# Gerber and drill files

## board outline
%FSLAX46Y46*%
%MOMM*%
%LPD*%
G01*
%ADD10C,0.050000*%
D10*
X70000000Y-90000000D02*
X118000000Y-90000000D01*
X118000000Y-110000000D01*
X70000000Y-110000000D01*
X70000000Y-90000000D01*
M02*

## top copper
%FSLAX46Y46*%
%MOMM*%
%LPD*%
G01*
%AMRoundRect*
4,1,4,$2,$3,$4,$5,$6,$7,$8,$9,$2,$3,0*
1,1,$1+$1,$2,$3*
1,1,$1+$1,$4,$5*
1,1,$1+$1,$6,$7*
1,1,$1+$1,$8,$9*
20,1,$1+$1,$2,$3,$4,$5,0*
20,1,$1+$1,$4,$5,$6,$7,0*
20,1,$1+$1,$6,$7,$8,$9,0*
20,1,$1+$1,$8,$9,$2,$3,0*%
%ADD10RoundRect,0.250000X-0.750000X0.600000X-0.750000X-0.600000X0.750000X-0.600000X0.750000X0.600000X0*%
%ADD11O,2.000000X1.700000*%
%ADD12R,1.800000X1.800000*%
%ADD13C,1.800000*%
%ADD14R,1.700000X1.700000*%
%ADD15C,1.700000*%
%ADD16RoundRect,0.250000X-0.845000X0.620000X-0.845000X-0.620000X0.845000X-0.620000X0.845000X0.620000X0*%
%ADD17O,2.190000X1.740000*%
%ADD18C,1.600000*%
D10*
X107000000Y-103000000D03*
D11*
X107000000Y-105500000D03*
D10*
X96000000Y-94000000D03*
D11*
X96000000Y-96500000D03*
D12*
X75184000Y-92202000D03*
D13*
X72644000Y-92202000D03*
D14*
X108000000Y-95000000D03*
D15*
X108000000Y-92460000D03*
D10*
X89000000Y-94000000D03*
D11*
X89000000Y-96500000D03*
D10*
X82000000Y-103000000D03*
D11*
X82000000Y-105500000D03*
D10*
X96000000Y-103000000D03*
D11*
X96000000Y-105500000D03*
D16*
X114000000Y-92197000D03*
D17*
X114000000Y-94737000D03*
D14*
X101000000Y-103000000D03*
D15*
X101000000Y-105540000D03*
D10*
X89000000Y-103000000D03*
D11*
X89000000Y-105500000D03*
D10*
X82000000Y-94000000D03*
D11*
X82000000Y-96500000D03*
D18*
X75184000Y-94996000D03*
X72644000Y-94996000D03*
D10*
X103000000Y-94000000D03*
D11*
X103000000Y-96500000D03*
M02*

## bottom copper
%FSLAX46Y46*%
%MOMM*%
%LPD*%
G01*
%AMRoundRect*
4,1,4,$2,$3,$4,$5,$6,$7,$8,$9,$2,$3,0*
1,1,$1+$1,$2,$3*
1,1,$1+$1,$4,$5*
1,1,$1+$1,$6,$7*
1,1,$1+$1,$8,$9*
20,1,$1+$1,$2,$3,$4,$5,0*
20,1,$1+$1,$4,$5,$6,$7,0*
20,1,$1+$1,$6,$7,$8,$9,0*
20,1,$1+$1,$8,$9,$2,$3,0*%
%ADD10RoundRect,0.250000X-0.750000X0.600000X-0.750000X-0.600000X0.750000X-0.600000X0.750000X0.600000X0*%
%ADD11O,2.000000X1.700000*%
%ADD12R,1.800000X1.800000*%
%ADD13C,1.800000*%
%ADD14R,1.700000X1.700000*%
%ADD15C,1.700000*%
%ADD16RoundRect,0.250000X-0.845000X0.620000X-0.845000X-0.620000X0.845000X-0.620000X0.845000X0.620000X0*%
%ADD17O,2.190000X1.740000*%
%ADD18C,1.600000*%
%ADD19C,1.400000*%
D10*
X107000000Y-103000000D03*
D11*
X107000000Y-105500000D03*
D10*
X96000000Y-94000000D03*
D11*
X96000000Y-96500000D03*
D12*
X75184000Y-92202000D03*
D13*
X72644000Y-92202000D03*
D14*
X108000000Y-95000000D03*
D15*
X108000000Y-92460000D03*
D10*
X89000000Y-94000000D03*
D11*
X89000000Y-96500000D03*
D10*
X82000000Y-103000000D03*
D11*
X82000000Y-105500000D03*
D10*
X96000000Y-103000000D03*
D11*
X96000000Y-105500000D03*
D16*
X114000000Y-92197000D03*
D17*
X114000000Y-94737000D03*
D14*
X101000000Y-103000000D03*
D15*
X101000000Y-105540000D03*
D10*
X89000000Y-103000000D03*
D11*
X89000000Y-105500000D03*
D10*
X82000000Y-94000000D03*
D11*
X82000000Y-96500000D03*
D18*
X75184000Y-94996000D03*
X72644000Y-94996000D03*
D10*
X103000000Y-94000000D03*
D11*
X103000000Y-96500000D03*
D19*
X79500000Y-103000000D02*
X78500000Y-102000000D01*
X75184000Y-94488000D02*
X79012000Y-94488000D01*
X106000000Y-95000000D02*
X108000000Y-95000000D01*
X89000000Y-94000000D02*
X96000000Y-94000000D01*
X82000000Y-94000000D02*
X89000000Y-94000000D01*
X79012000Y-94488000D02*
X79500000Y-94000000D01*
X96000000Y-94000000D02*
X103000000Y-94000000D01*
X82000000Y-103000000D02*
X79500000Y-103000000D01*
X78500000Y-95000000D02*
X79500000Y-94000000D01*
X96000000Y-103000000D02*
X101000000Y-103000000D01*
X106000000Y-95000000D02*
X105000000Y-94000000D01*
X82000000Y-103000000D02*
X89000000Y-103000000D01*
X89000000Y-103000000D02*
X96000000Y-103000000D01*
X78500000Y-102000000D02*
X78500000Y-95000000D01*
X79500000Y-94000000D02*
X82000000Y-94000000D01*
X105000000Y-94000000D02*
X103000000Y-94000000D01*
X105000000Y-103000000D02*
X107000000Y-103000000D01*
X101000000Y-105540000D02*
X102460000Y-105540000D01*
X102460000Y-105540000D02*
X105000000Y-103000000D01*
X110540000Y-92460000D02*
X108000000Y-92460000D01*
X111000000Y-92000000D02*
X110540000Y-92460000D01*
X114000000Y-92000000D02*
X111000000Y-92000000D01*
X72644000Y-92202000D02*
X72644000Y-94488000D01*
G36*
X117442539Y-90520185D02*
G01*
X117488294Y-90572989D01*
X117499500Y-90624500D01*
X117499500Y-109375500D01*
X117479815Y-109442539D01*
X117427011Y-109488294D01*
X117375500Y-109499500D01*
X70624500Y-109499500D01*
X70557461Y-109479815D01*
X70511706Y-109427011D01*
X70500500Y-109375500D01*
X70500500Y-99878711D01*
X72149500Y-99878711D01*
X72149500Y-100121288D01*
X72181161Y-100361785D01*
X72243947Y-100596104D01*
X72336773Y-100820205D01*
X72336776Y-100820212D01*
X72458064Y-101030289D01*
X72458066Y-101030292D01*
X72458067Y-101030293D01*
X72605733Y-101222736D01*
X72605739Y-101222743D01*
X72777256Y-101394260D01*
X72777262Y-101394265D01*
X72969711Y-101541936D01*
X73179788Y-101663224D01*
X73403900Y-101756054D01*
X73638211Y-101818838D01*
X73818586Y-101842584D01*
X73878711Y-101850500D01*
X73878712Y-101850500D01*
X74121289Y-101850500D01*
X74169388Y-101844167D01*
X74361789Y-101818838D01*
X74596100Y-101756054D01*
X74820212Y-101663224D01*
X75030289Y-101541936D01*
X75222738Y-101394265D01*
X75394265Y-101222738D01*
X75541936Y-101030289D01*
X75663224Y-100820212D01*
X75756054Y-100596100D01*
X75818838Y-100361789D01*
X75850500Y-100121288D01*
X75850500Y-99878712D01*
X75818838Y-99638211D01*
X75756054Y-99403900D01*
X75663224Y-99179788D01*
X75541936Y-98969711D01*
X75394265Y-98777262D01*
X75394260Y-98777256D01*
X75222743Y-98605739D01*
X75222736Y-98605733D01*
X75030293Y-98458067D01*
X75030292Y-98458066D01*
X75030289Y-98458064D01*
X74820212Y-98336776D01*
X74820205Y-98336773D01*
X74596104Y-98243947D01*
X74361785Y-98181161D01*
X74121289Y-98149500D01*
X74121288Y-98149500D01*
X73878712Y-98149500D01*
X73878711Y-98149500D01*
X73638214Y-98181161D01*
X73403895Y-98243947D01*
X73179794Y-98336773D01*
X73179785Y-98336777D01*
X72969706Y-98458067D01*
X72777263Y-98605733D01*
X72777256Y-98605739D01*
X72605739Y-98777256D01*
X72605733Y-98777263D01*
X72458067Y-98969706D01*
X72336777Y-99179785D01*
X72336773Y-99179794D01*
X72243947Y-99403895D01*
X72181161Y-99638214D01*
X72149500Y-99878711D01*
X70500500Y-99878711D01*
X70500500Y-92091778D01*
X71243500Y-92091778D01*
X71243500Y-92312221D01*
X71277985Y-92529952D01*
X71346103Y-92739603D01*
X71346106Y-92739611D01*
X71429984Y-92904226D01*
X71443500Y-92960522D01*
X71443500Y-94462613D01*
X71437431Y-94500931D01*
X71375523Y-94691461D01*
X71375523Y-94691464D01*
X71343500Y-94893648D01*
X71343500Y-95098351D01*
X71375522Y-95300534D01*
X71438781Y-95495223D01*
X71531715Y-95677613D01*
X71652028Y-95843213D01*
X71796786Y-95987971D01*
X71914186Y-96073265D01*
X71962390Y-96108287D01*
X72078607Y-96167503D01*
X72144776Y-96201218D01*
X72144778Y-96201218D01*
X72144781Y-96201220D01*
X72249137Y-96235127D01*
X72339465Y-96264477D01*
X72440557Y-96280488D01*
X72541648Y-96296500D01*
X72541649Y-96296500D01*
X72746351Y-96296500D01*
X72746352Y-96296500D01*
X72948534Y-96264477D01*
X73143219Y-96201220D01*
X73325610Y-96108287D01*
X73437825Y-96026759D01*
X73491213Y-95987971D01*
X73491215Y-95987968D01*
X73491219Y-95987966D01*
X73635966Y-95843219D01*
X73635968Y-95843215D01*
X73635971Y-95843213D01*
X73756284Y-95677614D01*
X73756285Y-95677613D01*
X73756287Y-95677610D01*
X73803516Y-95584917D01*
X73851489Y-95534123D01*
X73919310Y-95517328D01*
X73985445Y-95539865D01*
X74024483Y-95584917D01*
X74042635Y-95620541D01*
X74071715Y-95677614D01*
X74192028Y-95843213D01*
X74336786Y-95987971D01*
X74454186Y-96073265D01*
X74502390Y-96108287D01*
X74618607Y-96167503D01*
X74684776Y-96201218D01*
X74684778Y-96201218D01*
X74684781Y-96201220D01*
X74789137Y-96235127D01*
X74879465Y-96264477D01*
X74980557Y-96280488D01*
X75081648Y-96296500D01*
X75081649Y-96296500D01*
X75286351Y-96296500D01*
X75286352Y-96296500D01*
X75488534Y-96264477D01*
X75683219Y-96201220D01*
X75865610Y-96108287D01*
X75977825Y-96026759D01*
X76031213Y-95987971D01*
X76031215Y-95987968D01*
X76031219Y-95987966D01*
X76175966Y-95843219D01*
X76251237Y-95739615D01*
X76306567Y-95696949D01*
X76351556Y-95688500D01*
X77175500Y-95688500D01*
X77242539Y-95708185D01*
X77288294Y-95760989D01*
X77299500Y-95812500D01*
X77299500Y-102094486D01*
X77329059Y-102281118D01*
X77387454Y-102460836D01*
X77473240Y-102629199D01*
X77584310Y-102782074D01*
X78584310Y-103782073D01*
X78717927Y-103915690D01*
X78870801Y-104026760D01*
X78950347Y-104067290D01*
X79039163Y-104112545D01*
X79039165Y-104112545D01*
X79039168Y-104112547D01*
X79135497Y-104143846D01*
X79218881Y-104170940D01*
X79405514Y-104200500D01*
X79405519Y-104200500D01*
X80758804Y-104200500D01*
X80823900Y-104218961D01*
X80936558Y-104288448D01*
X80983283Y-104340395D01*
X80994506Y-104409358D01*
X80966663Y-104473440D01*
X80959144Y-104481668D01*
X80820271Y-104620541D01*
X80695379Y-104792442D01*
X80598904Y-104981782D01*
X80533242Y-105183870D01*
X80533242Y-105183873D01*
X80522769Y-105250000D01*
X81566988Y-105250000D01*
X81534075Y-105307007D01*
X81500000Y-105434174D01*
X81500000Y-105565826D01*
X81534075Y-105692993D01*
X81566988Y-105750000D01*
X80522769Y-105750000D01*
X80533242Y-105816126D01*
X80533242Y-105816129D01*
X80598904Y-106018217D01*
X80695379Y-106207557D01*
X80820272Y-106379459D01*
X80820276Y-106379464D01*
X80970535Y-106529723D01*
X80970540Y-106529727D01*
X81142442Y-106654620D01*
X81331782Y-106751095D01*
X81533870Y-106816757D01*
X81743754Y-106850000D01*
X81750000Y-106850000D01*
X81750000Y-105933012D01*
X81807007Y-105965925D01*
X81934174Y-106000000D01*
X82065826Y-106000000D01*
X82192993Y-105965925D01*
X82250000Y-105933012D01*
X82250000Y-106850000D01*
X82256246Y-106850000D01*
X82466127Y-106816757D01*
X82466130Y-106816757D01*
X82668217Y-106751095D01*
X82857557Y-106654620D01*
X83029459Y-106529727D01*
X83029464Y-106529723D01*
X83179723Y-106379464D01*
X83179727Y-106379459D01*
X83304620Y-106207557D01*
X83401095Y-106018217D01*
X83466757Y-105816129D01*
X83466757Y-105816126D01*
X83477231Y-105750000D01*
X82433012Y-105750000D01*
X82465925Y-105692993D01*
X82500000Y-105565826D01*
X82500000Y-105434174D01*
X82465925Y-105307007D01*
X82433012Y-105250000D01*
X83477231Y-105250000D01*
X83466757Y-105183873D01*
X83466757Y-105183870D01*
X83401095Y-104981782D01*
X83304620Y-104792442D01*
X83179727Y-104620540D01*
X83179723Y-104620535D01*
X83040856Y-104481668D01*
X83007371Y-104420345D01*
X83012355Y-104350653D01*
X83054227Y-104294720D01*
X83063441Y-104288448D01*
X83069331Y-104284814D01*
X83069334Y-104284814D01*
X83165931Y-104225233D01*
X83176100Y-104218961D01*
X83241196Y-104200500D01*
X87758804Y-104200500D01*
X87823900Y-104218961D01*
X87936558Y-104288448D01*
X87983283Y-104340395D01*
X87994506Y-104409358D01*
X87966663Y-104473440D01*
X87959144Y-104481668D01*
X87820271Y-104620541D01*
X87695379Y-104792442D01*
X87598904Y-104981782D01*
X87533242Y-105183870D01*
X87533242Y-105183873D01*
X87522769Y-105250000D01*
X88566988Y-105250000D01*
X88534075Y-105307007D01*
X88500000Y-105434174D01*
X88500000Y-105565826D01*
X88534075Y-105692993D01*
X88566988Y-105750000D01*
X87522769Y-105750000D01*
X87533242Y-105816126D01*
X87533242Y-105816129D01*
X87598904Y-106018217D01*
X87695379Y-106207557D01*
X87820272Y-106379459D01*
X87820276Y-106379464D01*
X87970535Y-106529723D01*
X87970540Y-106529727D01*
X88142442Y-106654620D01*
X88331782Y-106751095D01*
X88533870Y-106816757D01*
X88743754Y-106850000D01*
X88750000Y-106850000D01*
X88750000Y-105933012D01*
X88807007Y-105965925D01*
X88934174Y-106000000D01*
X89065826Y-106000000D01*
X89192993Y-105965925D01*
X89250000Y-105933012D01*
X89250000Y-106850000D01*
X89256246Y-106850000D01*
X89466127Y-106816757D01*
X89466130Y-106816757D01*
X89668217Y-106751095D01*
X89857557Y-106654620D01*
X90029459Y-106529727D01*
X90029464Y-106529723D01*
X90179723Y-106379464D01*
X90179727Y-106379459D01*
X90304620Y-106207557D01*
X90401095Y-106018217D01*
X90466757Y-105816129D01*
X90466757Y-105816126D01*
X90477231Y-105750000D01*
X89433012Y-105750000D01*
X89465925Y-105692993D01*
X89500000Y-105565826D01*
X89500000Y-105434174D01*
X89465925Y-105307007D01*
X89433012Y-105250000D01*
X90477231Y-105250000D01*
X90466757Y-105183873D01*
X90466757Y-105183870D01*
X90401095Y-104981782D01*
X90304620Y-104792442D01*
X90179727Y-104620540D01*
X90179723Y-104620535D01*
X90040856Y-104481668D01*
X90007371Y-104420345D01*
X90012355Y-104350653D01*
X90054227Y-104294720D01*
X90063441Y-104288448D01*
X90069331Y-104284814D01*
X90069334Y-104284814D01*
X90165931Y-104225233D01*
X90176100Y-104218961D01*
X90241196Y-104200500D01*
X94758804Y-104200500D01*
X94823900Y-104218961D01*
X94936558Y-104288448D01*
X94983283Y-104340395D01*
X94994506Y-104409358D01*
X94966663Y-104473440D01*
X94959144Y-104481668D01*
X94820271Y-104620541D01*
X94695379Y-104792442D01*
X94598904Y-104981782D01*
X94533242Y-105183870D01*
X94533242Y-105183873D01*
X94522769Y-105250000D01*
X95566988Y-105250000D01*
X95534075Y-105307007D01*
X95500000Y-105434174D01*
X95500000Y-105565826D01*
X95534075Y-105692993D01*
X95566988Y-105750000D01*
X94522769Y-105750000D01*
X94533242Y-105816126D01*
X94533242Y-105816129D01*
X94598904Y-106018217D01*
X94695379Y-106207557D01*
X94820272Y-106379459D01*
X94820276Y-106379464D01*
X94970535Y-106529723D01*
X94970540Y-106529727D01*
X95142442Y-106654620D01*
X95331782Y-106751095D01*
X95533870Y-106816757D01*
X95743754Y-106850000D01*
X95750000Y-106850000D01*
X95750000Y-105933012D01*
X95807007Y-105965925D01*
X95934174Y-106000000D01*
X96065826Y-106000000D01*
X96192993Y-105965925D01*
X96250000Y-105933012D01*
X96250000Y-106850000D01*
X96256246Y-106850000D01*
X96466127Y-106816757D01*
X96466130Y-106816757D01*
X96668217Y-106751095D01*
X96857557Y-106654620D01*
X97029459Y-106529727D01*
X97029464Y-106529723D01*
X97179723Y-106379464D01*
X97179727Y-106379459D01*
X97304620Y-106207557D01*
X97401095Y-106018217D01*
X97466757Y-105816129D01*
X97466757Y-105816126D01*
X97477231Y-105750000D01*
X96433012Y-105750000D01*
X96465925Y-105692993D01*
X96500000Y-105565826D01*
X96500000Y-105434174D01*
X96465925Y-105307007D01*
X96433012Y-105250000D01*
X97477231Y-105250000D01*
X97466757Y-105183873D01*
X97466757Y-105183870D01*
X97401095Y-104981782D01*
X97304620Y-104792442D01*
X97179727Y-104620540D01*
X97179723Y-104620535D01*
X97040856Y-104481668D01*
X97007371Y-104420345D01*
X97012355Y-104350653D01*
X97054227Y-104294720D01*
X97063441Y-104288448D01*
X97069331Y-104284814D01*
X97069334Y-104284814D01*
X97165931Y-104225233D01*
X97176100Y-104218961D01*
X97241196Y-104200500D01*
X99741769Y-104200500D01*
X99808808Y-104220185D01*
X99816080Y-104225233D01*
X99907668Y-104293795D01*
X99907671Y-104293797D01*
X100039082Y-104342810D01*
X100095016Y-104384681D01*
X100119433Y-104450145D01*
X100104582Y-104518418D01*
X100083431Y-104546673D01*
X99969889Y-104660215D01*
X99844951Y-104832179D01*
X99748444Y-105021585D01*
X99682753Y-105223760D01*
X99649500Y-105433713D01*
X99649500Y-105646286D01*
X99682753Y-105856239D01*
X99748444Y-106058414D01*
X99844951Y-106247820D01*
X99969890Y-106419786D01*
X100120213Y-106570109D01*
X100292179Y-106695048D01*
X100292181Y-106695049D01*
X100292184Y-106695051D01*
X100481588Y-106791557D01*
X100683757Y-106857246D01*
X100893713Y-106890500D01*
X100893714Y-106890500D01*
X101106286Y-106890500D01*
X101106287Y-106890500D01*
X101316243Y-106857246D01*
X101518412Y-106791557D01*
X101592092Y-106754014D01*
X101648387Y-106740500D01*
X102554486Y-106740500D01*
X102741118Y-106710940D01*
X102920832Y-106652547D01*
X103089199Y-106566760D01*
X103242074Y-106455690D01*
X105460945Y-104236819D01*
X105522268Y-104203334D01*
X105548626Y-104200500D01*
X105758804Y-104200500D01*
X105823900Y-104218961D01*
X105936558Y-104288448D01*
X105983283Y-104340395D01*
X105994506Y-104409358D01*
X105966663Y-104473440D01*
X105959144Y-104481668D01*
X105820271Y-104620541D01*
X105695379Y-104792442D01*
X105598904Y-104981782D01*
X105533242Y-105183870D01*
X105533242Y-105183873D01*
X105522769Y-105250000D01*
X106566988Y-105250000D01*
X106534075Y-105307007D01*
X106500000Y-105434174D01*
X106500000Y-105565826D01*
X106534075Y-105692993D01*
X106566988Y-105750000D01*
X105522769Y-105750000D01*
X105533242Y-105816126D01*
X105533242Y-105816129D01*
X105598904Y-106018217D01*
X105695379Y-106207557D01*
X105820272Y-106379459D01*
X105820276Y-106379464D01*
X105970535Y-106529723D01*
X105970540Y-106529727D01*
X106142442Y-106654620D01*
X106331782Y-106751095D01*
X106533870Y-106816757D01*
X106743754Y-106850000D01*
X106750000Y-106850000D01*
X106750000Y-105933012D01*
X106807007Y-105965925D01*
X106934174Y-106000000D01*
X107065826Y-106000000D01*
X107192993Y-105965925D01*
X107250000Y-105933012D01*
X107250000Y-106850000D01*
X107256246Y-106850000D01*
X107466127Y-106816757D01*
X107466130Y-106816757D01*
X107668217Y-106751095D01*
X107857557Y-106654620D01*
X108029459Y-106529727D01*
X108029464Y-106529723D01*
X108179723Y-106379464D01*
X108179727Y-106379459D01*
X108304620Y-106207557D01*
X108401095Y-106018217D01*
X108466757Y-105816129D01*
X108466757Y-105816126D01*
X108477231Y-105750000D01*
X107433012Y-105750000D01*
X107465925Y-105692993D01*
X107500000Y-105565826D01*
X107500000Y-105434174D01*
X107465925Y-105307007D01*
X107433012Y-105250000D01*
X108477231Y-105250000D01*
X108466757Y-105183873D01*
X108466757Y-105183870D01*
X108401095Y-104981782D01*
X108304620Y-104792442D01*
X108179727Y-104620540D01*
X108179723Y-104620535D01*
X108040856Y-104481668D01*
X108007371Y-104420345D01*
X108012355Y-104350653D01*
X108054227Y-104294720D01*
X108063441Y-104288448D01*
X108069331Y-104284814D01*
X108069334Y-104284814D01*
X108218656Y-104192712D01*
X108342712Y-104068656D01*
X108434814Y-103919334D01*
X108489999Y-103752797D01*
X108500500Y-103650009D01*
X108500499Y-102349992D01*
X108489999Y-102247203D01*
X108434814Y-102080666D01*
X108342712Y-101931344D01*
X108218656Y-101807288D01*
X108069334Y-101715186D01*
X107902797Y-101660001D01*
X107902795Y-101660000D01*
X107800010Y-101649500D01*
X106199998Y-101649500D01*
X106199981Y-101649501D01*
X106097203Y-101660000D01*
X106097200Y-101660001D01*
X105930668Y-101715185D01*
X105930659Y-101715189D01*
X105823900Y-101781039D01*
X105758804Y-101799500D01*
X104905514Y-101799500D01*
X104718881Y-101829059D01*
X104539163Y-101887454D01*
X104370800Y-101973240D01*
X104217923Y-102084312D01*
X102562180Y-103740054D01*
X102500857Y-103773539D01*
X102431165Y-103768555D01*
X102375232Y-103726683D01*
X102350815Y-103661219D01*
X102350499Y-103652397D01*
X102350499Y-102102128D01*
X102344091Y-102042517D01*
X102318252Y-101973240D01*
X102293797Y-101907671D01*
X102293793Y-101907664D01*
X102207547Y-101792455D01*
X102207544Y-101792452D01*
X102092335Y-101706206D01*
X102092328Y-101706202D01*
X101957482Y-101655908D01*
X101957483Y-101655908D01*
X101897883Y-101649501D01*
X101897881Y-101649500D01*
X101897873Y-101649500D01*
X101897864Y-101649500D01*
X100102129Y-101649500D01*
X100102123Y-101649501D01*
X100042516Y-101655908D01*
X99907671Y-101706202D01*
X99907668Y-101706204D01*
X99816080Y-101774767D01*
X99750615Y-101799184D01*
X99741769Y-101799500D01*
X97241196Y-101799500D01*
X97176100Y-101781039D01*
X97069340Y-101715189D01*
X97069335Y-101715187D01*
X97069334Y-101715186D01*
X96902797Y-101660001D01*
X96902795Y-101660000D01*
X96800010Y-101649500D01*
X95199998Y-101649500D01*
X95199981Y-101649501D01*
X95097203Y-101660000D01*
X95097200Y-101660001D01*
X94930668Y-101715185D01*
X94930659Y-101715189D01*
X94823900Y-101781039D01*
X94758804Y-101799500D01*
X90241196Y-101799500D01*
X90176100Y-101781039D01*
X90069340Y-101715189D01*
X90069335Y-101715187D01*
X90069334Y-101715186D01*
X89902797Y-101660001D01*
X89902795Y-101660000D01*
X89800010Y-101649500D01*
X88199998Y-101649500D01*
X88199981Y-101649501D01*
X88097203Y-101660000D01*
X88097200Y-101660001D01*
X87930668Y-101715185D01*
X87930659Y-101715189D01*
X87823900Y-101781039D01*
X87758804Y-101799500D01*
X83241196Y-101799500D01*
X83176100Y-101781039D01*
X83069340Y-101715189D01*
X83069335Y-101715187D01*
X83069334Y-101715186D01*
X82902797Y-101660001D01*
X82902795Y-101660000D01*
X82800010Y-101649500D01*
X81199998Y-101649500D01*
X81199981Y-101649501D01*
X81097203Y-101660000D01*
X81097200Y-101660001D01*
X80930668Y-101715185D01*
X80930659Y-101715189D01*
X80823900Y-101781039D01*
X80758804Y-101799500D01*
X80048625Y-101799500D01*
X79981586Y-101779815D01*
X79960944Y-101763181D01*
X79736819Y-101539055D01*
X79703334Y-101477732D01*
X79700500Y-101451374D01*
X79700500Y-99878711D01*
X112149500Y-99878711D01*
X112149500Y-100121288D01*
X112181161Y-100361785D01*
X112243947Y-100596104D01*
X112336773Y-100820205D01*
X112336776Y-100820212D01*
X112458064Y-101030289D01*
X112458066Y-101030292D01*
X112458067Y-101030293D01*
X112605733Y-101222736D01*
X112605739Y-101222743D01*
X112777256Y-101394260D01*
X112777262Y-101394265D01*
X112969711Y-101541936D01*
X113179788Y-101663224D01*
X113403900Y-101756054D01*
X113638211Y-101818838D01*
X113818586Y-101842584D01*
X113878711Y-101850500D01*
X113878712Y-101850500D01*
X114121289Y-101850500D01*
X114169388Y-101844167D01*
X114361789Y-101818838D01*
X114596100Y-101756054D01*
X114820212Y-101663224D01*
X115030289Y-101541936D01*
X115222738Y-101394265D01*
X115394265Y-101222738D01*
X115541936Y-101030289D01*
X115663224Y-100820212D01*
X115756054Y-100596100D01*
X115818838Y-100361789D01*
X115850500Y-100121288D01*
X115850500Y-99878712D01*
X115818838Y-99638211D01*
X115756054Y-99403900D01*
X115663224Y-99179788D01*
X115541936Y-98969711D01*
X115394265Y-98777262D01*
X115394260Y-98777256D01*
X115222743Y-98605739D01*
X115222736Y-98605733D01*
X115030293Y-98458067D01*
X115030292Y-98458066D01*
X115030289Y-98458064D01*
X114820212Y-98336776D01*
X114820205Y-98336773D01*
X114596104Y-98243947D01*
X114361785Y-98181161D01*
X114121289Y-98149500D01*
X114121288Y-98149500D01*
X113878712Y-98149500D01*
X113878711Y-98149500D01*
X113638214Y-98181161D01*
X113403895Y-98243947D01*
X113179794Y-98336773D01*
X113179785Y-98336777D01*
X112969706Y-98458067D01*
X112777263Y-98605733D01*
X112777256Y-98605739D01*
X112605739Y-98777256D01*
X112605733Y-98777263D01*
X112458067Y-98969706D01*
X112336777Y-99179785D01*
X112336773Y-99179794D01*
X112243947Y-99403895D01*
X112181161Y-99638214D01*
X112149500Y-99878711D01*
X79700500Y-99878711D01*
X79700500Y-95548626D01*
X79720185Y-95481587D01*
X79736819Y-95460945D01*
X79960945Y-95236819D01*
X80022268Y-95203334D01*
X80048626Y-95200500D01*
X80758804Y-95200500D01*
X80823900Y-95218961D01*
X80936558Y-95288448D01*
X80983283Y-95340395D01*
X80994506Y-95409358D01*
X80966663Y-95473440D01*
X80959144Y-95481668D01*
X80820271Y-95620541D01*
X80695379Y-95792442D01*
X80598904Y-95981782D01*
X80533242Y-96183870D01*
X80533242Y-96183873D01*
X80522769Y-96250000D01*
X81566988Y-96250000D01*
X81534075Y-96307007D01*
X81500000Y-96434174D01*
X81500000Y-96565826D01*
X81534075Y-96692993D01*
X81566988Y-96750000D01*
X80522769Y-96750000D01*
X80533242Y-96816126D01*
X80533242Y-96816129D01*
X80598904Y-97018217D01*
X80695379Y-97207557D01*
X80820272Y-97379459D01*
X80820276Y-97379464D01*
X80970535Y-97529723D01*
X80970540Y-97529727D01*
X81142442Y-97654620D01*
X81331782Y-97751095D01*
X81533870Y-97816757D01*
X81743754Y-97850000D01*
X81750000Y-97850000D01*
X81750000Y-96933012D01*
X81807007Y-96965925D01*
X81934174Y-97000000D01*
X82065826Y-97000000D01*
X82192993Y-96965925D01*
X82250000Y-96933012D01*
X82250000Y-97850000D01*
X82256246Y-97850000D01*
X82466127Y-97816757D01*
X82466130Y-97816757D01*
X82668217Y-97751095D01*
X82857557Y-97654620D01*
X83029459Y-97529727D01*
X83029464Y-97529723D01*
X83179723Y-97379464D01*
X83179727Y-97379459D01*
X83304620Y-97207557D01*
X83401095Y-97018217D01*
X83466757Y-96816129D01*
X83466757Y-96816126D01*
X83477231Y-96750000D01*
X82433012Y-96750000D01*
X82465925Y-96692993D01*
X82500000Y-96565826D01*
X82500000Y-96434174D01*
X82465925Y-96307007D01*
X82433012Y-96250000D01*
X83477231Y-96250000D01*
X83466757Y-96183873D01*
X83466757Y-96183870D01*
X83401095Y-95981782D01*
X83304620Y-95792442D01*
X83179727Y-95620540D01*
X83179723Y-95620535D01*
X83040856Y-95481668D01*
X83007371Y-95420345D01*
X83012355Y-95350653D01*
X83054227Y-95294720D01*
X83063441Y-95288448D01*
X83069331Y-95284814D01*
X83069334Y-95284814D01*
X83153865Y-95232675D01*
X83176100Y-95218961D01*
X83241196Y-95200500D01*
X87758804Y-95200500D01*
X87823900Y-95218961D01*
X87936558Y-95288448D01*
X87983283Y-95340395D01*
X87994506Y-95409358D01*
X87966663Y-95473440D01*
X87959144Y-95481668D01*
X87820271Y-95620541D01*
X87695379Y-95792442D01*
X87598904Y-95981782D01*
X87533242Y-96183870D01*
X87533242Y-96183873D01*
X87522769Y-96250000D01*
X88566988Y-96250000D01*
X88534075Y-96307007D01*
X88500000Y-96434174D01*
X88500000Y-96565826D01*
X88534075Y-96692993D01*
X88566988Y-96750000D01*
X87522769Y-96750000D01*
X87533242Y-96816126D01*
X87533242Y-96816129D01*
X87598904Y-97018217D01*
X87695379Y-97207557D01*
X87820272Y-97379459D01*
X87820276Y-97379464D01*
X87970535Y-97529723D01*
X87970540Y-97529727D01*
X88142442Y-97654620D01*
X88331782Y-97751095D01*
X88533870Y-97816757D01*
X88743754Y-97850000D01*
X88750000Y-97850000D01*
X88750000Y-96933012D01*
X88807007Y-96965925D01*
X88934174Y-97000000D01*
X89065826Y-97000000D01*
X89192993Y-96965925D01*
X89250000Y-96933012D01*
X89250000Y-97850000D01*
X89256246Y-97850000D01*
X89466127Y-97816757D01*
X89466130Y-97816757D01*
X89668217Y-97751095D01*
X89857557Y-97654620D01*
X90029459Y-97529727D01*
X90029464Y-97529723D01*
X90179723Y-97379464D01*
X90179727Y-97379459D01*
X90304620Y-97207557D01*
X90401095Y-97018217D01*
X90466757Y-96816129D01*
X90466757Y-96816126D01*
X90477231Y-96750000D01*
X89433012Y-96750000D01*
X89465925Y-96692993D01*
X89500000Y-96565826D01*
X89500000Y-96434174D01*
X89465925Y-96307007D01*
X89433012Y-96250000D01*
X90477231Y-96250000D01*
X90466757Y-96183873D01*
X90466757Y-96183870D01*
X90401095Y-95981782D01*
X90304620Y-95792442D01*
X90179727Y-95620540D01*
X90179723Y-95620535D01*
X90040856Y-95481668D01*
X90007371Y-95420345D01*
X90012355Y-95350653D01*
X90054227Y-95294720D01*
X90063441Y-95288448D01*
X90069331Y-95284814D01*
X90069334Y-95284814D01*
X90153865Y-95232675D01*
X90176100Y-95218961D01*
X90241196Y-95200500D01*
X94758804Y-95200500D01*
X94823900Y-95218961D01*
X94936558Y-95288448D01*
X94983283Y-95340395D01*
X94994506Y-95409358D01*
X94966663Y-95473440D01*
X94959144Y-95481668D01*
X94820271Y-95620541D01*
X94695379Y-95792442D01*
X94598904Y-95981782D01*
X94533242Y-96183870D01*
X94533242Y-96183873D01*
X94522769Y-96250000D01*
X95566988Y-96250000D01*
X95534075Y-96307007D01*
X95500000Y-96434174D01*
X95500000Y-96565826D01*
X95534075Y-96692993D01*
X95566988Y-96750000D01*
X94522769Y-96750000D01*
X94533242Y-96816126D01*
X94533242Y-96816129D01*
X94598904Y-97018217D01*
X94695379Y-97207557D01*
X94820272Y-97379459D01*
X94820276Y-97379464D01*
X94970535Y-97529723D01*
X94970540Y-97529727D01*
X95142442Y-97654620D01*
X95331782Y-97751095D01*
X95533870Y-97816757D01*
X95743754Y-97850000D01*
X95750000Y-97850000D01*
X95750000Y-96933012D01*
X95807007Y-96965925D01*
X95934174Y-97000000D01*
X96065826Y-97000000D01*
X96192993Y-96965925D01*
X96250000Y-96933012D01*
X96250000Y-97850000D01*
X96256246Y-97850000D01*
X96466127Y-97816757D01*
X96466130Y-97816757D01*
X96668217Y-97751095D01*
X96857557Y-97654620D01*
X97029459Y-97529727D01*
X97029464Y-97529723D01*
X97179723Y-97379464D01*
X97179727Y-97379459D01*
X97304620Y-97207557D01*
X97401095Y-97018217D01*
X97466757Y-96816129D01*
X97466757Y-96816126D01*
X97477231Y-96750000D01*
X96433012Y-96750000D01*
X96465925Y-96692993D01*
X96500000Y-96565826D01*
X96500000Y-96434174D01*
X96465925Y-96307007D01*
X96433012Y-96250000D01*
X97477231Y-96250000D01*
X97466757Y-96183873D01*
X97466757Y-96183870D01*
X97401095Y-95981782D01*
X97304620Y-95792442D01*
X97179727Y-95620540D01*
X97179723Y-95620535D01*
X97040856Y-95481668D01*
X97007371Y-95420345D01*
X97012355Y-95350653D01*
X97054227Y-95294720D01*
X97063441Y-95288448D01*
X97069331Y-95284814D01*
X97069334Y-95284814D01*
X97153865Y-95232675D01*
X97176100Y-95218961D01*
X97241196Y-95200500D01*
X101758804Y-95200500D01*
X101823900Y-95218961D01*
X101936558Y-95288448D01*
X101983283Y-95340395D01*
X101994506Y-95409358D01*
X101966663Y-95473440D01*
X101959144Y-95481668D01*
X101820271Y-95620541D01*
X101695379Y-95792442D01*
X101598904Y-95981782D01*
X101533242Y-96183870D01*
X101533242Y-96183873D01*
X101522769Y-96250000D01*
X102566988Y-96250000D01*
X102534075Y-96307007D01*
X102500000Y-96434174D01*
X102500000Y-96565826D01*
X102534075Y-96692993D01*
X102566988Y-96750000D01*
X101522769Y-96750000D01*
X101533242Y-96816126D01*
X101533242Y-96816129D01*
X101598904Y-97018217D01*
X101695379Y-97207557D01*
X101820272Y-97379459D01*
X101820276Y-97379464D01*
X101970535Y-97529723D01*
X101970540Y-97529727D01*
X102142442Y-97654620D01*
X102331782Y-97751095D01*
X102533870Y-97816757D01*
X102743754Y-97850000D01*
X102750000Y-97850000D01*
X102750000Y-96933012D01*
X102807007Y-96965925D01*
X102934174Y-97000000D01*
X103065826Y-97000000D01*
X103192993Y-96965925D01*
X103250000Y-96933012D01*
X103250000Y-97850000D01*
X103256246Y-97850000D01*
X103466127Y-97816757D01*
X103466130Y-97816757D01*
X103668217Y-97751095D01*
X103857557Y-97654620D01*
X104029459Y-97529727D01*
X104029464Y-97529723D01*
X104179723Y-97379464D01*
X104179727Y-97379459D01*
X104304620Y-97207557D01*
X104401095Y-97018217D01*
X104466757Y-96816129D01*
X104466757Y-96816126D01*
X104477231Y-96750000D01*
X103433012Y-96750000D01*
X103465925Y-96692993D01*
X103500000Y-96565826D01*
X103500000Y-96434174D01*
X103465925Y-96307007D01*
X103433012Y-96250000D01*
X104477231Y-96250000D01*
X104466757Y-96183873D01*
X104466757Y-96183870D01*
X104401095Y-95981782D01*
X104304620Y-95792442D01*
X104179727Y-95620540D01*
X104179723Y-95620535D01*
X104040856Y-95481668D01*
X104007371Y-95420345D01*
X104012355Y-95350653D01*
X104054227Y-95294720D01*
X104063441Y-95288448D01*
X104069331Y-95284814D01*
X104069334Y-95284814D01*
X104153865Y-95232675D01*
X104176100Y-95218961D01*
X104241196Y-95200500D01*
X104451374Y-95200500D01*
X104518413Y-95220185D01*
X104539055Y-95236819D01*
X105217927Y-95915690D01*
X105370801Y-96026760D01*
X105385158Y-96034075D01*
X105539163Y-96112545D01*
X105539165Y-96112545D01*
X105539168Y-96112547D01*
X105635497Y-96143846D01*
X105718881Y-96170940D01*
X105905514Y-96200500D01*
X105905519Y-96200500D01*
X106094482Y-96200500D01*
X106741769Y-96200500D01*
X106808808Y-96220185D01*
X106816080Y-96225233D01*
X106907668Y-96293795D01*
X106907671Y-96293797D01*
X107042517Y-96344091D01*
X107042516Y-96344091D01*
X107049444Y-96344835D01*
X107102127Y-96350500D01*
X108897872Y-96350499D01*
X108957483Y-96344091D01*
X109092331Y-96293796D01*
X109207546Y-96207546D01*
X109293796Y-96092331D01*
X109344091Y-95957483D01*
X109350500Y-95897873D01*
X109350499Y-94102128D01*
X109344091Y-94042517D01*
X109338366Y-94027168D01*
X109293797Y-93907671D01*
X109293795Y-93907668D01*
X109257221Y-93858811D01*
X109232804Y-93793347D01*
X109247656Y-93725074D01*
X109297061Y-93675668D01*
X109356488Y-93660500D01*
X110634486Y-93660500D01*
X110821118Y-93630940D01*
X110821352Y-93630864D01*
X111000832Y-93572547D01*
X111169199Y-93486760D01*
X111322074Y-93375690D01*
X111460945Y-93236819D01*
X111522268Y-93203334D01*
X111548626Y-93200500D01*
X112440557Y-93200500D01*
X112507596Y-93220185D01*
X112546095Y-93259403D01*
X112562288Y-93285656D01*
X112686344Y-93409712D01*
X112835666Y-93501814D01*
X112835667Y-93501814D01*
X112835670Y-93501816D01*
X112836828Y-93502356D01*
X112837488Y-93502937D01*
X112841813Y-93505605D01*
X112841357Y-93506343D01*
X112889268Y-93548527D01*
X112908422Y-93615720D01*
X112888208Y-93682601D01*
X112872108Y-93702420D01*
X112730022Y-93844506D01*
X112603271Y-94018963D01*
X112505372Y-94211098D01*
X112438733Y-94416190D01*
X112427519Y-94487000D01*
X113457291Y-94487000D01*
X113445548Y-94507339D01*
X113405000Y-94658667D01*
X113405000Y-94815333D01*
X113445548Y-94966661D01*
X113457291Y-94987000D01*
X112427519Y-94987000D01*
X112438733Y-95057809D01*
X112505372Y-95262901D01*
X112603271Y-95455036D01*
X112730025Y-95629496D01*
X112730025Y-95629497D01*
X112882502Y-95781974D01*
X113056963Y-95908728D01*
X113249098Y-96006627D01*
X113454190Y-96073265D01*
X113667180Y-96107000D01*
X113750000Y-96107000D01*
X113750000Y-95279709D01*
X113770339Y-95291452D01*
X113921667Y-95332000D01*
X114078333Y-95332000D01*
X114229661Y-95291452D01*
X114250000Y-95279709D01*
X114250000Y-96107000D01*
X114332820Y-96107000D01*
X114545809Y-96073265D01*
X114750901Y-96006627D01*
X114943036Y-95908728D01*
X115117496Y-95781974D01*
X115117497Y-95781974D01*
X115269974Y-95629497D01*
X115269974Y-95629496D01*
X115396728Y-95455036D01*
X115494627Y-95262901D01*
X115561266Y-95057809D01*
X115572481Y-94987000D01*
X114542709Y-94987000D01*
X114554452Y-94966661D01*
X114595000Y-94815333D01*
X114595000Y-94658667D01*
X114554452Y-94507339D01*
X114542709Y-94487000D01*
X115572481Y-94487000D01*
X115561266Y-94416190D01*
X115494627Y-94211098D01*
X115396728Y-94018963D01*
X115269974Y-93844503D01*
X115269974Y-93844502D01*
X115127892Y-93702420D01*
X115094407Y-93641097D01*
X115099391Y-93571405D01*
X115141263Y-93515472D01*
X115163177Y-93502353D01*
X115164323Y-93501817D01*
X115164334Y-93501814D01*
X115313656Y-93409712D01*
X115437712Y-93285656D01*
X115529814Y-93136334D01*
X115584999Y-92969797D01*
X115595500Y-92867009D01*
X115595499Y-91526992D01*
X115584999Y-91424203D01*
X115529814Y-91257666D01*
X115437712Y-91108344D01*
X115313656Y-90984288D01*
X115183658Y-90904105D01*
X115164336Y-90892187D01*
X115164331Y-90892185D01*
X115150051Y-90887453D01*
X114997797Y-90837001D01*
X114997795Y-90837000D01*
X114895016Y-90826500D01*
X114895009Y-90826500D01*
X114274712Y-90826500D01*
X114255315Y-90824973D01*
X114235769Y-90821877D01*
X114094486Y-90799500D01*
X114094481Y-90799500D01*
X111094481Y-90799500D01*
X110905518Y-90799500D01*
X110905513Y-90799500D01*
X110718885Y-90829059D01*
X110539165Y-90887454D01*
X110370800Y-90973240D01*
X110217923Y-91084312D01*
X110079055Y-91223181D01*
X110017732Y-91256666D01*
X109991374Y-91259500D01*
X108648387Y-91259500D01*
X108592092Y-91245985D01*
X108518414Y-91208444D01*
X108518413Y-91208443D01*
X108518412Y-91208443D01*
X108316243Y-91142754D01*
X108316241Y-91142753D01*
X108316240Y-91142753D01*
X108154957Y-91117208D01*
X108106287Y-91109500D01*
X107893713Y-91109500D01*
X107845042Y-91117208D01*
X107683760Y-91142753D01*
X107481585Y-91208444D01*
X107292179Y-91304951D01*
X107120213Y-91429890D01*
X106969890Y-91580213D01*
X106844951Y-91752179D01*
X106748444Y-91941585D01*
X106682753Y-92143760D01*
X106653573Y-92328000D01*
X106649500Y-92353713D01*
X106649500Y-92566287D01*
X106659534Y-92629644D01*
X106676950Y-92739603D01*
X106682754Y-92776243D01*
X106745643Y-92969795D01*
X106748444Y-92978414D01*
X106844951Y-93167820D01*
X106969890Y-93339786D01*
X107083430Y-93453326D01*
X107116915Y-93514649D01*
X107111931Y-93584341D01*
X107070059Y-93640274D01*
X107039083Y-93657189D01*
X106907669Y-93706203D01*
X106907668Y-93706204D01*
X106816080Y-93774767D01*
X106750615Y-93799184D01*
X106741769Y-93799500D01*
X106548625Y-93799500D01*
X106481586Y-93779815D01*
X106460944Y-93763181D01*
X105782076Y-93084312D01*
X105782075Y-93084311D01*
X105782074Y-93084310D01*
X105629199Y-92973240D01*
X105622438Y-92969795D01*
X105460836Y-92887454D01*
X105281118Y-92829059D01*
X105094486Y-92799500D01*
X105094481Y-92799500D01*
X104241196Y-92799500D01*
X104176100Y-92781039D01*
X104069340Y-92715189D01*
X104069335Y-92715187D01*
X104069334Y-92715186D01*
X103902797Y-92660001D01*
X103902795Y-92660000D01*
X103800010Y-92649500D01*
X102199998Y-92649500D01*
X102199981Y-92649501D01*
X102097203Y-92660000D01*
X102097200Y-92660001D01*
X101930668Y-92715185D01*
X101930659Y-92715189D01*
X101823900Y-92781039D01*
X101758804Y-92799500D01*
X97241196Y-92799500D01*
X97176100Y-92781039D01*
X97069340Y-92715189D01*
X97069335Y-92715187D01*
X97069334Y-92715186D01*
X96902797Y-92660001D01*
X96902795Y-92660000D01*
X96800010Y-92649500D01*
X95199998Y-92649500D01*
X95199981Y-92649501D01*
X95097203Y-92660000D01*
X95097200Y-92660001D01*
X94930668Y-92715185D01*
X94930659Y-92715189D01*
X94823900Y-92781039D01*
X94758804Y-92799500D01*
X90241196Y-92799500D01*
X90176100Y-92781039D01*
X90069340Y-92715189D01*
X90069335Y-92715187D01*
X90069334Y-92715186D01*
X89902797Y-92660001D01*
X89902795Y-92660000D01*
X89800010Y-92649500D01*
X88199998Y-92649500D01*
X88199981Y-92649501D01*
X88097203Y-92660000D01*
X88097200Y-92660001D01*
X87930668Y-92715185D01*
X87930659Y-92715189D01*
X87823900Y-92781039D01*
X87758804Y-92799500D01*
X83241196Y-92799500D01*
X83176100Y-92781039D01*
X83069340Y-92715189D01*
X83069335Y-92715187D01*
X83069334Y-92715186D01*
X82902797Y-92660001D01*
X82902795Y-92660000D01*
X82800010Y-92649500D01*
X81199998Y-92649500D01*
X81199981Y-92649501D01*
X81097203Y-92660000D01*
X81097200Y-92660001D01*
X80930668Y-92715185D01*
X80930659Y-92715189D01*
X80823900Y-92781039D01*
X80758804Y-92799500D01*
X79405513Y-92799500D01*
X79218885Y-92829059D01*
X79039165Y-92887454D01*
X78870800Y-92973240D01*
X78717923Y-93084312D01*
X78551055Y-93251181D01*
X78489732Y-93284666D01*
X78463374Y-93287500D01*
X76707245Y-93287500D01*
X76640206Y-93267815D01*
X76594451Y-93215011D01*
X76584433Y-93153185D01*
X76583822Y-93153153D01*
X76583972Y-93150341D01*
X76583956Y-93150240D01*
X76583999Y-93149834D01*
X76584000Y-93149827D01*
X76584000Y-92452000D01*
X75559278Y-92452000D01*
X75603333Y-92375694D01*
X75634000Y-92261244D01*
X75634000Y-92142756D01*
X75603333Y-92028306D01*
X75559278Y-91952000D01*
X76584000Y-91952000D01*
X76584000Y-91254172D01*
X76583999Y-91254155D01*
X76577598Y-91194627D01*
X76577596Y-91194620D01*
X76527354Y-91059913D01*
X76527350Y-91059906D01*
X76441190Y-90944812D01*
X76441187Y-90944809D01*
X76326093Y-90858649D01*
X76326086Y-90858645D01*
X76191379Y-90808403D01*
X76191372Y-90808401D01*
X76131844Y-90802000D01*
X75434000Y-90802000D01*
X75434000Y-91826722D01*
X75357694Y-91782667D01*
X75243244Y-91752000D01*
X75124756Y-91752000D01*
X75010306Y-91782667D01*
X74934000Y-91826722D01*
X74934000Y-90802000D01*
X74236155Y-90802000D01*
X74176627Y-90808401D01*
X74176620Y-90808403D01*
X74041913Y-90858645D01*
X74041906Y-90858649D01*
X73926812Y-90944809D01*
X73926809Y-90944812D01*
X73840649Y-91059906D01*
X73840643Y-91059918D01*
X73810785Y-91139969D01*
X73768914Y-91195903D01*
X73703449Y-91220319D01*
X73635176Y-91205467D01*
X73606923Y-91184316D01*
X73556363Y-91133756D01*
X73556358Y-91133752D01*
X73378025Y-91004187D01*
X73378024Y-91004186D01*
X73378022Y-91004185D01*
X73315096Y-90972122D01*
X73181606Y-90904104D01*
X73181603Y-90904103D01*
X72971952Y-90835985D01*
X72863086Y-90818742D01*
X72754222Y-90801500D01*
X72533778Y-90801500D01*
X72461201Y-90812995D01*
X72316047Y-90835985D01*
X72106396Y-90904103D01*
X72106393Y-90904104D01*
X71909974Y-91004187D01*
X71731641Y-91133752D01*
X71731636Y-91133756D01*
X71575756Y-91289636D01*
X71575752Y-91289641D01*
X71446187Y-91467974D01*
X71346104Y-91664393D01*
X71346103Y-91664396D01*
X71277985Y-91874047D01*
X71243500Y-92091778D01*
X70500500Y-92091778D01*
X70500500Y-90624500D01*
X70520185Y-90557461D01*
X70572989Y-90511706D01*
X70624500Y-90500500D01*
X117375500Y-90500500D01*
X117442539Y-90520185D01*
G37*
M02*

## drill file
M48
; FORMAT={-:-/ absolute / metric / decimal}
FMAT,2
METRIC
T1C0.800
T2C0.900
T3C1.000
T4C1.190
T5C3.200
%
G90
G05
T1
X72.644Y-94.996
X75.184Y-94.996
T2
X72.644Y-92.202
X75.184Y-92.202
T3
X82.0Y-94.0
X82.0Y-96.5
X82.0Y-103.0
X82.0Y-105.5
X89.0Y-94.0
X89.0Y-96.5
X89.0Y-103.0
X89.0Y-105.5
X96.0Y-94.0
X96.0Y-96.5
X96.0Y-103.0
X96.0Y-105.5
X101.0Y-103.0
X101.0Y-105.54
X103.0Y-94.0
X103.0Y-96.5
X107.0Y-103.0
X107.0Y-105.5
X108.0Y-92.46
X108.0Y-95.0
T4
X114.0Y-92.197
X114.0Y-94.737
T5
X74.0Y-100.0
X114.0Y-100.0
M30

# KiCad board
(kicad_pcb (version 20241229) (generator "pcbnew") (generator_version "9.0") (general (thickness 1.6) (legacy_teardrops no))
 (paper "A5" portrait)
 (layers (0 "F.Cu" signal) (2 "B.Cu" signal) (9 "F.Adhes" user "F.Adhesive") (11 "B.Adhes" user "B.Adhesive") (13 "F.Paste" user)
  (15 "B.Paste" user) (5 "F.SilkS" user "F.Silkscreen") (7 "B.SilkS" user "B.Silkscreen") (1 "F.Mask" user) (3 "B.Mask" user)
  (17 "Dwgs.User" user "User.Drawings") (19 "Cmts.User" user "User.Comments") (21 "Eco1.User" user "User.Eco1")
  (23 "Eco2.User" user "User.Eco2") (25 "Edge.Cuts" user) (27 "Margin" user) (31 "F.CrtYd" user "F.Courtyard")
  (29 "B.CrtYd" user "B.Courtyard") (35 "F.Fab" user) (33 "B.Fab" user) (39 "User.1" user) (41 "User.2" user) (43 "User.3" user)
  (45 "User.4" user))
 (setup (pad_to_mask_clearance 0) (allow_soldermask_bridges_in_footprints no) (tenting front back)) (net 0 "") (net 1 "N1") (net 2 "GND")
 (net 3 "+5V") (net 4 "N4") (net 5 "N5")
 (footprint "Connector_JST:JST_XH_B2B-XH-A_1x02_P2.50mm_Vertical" (layer "F.Cu") (at 107 103 -90)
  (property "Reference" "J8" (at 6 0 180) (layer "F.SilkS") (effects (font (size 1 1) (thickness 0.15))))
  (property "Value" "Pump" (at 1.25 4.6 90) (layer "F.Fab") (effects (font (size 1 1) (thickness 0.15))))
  (pad "1" thru_hole roundrect (at 0 0 270) (size 1.7 2) (drill 1) (layers "*.Cu" "*.Mask") (remove_unused_layers no)
   (roundrect_rratio 0.147059) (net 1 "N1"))
  (pad "2" thru_hole oval (at 2.5 0 270) (size 1.7 2) (drill 1) (layers "*.Cu" "*.Mask") (remove_unused_layers no) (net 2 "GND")))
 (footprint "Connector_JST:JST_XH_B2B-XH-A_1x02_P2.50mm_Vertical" (layer "F.Cu") (at 96 94 -90)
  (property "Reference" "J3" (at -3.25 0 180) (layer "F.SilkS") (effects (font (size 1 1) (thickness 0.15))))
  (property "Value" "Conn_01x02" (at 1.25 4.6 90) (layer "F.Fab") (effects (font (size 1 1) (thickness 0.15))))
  (pad "1" thru_hole roundrect (at 0 0 270) (size 1.7 2) (drill 1) (layers "*.Cu" "*.Mask") (remove_unused_layers no)
   (roundrect_rratio 0.147059) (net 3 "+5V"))
  (pad "2" thru_hole oval (at 2.5 0 270) (size 1.7 2) (drill 1) (layers "*.Cu" "*.Mask") (remove_unused_layers no) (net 2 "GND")))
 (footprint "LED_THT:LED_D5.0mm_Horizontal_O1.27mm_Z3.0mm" (layer "F.Cu") (at 75.184 92.202 180)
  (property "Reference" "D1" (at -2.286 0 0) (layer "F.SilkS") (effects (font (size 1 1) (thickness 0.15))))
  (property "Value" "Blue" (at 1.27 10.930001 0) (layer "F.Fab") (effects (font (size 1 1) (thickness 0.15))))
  (pad "1" thru_hole rect (at 0 0 180) (size 1.8 1.8) (drill 0.9) (layers "*.Cu" "*.Mask") (remove_unused_layers no) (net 2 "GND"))
  (pad "2" thru_hole circle (at 2.54 0 180) (size 1.8 1.8) (drill 0.9) (layers "*.Cu" "*.Mask") (remove_unused_layers no) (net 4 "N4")))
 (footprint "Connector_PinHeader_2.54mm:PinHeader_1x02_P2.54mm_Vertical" (layer "F.Cu") (at 108 95 180)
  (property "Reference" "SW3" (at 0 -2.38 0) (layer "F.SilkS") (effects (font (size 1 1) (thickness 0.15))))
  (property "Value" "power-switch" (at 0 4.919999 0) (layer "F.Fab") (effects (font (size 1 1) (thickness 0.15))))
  (pad "1" thru_hole rect (at 0 0 180) (size 1.7 1.7) (drill 1) (layers "*.Cu" "*.Mask") (remove_unused_layers no) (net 3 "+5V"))
  (pad "2" thru_hole circle (at 0 2.54 180) (size 1.7 1.7) (drill 1) (layers "*.Cu" "*.Mask") (remove_unused_layers no) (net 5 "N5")))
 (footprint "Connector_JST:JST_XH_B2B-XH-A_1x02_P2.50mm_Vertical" (layer "F.Cu") (at 89 94 -90)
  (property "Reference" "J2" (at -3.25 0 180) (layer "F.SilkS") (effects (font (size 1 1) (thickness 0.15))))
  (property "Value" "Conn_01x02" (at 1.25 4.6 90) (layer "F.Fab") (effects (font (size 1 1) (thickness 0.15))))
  (pad "1" thru_hole roundrect (at 0 0 270) (size 1.7 2) (drill 1) (layers "*.Cu" "*.Mask") (remove_unused_layers no)
   (roundrect_rratio 0.147059) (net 3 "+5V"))
  (pad "2" thru_hole oval (at 2.5 0 270) (size 1.7 2) (drill 1) (layers "*.Cu" "*.Mask") (remove_unused_layers no) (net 2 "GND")))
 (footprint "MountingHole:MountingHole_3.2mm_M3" (layer "F.Cu") (at 114 100)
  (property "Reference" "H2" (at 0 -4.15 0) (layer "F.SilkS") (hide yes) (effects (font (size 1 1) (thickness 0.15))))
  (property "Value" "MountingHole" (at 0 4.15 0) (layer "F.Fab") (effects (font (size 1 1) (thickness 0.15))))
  (pad "" np_thru_hole circle (at 0 0) (size 3.2 3.2) (drill 3.2) (layers "*.Cu" "*.Mask")))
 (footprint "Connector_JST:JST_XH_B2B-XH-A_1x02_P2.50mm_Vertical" (layer "F.Cu") (at 82 103 -90)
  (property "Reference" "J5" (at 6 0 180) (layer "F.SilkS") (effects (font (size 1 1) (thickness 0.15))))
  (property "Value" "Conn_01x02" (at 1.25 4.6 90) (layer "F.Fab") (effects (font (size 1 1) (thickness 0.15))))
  (pad "1" thru_hole roundrect (at 0 0 270) (size 1.7 2) (drill 1) (layers "*.Cu" "*.Mask") (remove_unused_layers no)
   (roundrect_rratio 0.147059) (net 3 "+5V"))
  (pad "2" thru_hole oval (at 2.5 0 270) (size 1.7 2) (drill 1) (layers "*.Cu" "*.Mask") (remove_unused_layers no) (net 2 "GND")))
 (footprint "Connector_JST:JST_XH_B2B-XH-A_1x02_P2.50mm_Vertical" (layer "F.Cu") (at 96 103 -90)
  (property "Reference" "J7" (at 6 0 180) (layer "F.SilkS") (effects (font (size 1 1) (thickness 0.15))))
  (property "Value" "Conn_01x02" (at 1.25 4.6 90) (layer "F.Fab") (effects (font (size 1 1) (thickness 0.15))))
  (pad "1" thru_hole roundrect (at 0 0 270) (size 1.7 2) (drill 1) (layers "*.Cu" "*.Mask") (remove_unused_layers no)
   (roundrect_rratio 0.147059) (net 3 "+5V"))
  (pad "2" thru_hole oval (at 2.5 0 270) (size 1.7 2) (drill 1) (layers "*.Cu" "*.Mask") (remove_unused_layers no) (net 2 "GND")))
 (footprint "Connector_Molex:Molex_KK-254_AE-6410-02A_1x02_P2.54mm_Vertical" (layer "F.Cu") (at 114 92.197 -90)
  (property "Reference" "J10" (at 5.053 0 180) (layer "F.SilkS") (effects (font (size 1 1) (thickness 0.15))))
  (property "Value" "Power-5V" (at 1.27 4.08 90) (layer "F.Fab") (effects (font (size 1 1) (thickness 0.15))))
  (pad "1" thru_hole roundrect (at 0 0 270) (size 1.74 2.19) (drill 1.19) (layers "*.Cu" "*.Mask") (remove_unused_layers no)
   (roundrect_rratio 0.143678) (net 5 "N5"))
  (pad "2" thru_hole oval (at 2.54 0 270) (size 1.74 2.19) (drill 1.19) (layers "*.Cu" "*.Mask") (remove_unused_layers no) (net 2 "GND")))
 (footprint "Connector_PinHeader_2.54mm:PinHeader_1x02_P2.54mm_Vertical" (layer "F.Cu") (at 101 103)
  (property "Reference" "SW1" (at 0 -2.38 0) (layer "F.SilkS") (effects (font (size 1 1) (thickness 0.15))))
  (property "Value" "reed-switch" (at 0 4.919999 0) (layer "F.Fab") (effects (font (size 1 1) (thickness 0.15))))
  (pad "1" thru_hole rect (at 0 0) (size 1.7 1.7) (drill 1) (layers "*.Cu" "*.Mask") (remove_unused_layers no) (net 3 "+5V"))
  (pad "2" thru_hole circle (at 0 2.54) (size 1.7 1.7) (drill 1) (layers "*.Cu" "*.Mask") (remove_unused_layers no) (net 1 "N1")))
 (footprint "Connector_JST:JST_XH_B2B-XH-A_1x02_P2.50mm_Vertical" (layer "F.Cu") (at 89 103 -90)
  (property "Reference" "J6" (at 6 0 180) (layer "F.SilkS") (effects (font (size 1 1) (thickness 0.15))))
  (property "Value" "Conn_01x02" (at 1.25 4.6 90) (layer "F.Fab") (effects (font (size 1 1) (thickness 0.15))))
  (pad "1" thru_hole roundrect (at 0 0 270) (size 1.7 2) (drill 1) (layers "*.Cu" "*.Mask") (remove_unused_layers no)
   (roundrect_rratio 0.147059) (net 3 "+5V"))
  (pad "2" thru_hole oval (at 2.5 0 270) (size 1.7 2) (drill 1) (layers "*.Cu" "*.Mask") (remove_unused_layers no) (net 2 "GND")))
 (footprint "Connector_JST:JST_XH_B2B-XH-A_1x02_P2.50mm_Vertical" (layer "F.Cu") (at 82 94 -90)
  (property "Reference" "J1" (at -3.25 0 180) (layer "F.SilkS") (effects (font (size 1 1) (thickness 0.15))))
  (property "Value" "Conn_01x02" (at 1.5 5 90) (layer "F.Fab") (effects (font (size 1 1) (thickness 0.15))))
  (pad "1" thru_hole roundrect (at 0 0 270) (size 1.7 2) (drill 1) (layers "*.Cu" "*.Mask") (remove_unused_layers no)
   (roundrect_rratio 0.147059) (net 3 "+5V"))
  (pad "2" thru_hole oval (at 2.5 0 270) (size 1.7 2) (drill 1) (layers "*.Cu" "*.Mask") (remove_unused_layers no) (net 2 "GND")))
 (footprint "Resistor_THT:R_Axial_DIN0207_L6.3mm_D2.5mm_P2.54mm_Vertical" (layer "F.Cu") (at 75.184 94.996 180)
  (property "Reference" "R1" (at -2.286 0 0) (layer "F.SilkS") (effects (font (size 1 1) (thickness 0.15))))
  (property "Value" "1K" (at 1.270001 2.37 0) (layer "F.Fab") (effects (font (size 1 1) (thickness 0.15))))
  (pad "1" thru_hole circle (at 0 0 180) (size 1.6 1.6) (drill 0.8) (layers "*.Cu" "*.Mask") (remove_unused_layers no) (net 3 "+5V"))
  (pad "2" thru_hole circle (at 2.54 0 180) (size 1.6 1.6) (drill 0.8) (layers "*.Cu" "*.Mask") (remove_unused_layers no) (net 4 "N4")))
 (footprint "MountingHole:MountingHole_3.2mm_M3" (layer "F.Cu") (at 74 100)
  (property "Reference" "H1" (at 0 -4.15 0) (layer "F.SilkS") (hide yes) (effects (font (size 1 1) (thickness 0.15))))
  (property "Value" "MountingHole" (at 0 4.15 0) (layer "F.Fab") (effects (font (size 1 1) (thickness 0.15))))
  (pad "" np_thru_hole circle (at 0 0) (size 3.2 3.2) (drill 3.2) (layers "*.Cu" "*.Mask")))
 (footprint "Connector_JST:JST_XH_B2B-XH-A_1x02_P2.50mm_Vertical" (layer "F.Cu") (at 103 94 -90)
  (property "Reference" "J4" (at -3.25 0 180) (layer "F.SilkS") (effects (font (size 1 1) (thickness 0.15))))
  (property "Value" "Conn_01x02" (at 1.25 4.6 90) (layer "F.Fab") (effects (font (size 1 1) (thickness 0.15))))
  (pad "1" thru_hole roundrect (at 0 0 270) (size 1.7 2) (drill 1) (layers "*.Cu" "*.Mask") (remove_unused_layers no)
   (roundrect_rratio 0.147059) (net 3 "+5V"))
  (pad "2" thru_hole oval (at 2.5 0 270) (size 1.7 2) (drill 1) (layers "*.Cu" "*.Mask") (remove_unused_layers no) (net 2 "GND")))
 (gr_rect (start 70 90) (end 118 110) (stroke (width 0.05) (type default)) (fill no) (layer "Edge.Cuts"))
 (segment (start 79.5 103) (end 78.5 102) (width 1.4) (layer "B.Cu") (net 3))
 (segment (start 75.184 94.488) (end 79.012 94.488) (width 1.4) (layer "B.Cu") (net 3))
 (segment (start 106 95) (end 108 95) (width 1.4) (layer "B.Cu") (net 3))
 (segment (start 89 94) (end 96 94) (width 1.4) (layer "B.Cu") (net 3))
 (segment (start 82 94) (end 89 94) (width 1.4) (layer "B.Cu") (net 3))
 (segment (start 79.012 94.488) (end 79.5 94) (width 1.4) (layer "B.Cu") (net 3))
 (segment (start 96 94) (end 103 94) (width 1.4) (layer "B.Cu") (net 3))
 (segment (start 82 103) (end 79.5 103) (width 1.4) (layer "B.Cu") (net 3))
 (segment (start 78.5 95) (end 79.5 94) (width 1.4) (layer "B.Cu") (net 3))
 (segment (start 96 103) (end 101 103) (width 1.4) (layer "B.Cu") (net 3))
 (segment (start 106 95) (end 105 94) (width 1.4) (layer "B.Cu") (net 3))
 (segment (start 82 103) (end 89 103) (width 1.4) (layer "B.Cu") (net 3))
 (segment (start 89 103) (end 96 103) (width 1.4) (layer "B.Cu") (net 3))
 (segment (start 78.5 102) (end 78.5 95) (width 1.4) (layer "B.Cu") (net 3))
 (segment (start 79.5 94) (end 82 94) (width 1.4) (layer "B.Cu") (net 3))
 (segment (start 105 94) (end 103 94) (width 1.4) (layer "B.Cu") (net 3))
 (segment (start 105 103) (end 107 103) (width 1.4) (layer "B.Cu") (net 1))
 (segment (start 101 105.54) (end 102.46 105.54) (width 1.4) (layer "B.Cu") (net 1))
 (segment (start 102.46 105.54) (end 105 103) (width 1.4) (layer "B.Cu") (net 1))
 (segment (start 110.54 92.46) (end 108 92.46) (width 1.4) (layer "B.Cu") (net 5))
 (segment (start 111 92) (end 110.54 92.46) (width 1.4) (layer "B.Cu") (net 5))
 (segment (start 114 92) (end 111 92) (width 1.4) (layer "B.Cu") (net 5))
 (segment (start 72.644 92.202) (end 72.644 94.488) (width 1.4) (layer "B.Cu") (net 4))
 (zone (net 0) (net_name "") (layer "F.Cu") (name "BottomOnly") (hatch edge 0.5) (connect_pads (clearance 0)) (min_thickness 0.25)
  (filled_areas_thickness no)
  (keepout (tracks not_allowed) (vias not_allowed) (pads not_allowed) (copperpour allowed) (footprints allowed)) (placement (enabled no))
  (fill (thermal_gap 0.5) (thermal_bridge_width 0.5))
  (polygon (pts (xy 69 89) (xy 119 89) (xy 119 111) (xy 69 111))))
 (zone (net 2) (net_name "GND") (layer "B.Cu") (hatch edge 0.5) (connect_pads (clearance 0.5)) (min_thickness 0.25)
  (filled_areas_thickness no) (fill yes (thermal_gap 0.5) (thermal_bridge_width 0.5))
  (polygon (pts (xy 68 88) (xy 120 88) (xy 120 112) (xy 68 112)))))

